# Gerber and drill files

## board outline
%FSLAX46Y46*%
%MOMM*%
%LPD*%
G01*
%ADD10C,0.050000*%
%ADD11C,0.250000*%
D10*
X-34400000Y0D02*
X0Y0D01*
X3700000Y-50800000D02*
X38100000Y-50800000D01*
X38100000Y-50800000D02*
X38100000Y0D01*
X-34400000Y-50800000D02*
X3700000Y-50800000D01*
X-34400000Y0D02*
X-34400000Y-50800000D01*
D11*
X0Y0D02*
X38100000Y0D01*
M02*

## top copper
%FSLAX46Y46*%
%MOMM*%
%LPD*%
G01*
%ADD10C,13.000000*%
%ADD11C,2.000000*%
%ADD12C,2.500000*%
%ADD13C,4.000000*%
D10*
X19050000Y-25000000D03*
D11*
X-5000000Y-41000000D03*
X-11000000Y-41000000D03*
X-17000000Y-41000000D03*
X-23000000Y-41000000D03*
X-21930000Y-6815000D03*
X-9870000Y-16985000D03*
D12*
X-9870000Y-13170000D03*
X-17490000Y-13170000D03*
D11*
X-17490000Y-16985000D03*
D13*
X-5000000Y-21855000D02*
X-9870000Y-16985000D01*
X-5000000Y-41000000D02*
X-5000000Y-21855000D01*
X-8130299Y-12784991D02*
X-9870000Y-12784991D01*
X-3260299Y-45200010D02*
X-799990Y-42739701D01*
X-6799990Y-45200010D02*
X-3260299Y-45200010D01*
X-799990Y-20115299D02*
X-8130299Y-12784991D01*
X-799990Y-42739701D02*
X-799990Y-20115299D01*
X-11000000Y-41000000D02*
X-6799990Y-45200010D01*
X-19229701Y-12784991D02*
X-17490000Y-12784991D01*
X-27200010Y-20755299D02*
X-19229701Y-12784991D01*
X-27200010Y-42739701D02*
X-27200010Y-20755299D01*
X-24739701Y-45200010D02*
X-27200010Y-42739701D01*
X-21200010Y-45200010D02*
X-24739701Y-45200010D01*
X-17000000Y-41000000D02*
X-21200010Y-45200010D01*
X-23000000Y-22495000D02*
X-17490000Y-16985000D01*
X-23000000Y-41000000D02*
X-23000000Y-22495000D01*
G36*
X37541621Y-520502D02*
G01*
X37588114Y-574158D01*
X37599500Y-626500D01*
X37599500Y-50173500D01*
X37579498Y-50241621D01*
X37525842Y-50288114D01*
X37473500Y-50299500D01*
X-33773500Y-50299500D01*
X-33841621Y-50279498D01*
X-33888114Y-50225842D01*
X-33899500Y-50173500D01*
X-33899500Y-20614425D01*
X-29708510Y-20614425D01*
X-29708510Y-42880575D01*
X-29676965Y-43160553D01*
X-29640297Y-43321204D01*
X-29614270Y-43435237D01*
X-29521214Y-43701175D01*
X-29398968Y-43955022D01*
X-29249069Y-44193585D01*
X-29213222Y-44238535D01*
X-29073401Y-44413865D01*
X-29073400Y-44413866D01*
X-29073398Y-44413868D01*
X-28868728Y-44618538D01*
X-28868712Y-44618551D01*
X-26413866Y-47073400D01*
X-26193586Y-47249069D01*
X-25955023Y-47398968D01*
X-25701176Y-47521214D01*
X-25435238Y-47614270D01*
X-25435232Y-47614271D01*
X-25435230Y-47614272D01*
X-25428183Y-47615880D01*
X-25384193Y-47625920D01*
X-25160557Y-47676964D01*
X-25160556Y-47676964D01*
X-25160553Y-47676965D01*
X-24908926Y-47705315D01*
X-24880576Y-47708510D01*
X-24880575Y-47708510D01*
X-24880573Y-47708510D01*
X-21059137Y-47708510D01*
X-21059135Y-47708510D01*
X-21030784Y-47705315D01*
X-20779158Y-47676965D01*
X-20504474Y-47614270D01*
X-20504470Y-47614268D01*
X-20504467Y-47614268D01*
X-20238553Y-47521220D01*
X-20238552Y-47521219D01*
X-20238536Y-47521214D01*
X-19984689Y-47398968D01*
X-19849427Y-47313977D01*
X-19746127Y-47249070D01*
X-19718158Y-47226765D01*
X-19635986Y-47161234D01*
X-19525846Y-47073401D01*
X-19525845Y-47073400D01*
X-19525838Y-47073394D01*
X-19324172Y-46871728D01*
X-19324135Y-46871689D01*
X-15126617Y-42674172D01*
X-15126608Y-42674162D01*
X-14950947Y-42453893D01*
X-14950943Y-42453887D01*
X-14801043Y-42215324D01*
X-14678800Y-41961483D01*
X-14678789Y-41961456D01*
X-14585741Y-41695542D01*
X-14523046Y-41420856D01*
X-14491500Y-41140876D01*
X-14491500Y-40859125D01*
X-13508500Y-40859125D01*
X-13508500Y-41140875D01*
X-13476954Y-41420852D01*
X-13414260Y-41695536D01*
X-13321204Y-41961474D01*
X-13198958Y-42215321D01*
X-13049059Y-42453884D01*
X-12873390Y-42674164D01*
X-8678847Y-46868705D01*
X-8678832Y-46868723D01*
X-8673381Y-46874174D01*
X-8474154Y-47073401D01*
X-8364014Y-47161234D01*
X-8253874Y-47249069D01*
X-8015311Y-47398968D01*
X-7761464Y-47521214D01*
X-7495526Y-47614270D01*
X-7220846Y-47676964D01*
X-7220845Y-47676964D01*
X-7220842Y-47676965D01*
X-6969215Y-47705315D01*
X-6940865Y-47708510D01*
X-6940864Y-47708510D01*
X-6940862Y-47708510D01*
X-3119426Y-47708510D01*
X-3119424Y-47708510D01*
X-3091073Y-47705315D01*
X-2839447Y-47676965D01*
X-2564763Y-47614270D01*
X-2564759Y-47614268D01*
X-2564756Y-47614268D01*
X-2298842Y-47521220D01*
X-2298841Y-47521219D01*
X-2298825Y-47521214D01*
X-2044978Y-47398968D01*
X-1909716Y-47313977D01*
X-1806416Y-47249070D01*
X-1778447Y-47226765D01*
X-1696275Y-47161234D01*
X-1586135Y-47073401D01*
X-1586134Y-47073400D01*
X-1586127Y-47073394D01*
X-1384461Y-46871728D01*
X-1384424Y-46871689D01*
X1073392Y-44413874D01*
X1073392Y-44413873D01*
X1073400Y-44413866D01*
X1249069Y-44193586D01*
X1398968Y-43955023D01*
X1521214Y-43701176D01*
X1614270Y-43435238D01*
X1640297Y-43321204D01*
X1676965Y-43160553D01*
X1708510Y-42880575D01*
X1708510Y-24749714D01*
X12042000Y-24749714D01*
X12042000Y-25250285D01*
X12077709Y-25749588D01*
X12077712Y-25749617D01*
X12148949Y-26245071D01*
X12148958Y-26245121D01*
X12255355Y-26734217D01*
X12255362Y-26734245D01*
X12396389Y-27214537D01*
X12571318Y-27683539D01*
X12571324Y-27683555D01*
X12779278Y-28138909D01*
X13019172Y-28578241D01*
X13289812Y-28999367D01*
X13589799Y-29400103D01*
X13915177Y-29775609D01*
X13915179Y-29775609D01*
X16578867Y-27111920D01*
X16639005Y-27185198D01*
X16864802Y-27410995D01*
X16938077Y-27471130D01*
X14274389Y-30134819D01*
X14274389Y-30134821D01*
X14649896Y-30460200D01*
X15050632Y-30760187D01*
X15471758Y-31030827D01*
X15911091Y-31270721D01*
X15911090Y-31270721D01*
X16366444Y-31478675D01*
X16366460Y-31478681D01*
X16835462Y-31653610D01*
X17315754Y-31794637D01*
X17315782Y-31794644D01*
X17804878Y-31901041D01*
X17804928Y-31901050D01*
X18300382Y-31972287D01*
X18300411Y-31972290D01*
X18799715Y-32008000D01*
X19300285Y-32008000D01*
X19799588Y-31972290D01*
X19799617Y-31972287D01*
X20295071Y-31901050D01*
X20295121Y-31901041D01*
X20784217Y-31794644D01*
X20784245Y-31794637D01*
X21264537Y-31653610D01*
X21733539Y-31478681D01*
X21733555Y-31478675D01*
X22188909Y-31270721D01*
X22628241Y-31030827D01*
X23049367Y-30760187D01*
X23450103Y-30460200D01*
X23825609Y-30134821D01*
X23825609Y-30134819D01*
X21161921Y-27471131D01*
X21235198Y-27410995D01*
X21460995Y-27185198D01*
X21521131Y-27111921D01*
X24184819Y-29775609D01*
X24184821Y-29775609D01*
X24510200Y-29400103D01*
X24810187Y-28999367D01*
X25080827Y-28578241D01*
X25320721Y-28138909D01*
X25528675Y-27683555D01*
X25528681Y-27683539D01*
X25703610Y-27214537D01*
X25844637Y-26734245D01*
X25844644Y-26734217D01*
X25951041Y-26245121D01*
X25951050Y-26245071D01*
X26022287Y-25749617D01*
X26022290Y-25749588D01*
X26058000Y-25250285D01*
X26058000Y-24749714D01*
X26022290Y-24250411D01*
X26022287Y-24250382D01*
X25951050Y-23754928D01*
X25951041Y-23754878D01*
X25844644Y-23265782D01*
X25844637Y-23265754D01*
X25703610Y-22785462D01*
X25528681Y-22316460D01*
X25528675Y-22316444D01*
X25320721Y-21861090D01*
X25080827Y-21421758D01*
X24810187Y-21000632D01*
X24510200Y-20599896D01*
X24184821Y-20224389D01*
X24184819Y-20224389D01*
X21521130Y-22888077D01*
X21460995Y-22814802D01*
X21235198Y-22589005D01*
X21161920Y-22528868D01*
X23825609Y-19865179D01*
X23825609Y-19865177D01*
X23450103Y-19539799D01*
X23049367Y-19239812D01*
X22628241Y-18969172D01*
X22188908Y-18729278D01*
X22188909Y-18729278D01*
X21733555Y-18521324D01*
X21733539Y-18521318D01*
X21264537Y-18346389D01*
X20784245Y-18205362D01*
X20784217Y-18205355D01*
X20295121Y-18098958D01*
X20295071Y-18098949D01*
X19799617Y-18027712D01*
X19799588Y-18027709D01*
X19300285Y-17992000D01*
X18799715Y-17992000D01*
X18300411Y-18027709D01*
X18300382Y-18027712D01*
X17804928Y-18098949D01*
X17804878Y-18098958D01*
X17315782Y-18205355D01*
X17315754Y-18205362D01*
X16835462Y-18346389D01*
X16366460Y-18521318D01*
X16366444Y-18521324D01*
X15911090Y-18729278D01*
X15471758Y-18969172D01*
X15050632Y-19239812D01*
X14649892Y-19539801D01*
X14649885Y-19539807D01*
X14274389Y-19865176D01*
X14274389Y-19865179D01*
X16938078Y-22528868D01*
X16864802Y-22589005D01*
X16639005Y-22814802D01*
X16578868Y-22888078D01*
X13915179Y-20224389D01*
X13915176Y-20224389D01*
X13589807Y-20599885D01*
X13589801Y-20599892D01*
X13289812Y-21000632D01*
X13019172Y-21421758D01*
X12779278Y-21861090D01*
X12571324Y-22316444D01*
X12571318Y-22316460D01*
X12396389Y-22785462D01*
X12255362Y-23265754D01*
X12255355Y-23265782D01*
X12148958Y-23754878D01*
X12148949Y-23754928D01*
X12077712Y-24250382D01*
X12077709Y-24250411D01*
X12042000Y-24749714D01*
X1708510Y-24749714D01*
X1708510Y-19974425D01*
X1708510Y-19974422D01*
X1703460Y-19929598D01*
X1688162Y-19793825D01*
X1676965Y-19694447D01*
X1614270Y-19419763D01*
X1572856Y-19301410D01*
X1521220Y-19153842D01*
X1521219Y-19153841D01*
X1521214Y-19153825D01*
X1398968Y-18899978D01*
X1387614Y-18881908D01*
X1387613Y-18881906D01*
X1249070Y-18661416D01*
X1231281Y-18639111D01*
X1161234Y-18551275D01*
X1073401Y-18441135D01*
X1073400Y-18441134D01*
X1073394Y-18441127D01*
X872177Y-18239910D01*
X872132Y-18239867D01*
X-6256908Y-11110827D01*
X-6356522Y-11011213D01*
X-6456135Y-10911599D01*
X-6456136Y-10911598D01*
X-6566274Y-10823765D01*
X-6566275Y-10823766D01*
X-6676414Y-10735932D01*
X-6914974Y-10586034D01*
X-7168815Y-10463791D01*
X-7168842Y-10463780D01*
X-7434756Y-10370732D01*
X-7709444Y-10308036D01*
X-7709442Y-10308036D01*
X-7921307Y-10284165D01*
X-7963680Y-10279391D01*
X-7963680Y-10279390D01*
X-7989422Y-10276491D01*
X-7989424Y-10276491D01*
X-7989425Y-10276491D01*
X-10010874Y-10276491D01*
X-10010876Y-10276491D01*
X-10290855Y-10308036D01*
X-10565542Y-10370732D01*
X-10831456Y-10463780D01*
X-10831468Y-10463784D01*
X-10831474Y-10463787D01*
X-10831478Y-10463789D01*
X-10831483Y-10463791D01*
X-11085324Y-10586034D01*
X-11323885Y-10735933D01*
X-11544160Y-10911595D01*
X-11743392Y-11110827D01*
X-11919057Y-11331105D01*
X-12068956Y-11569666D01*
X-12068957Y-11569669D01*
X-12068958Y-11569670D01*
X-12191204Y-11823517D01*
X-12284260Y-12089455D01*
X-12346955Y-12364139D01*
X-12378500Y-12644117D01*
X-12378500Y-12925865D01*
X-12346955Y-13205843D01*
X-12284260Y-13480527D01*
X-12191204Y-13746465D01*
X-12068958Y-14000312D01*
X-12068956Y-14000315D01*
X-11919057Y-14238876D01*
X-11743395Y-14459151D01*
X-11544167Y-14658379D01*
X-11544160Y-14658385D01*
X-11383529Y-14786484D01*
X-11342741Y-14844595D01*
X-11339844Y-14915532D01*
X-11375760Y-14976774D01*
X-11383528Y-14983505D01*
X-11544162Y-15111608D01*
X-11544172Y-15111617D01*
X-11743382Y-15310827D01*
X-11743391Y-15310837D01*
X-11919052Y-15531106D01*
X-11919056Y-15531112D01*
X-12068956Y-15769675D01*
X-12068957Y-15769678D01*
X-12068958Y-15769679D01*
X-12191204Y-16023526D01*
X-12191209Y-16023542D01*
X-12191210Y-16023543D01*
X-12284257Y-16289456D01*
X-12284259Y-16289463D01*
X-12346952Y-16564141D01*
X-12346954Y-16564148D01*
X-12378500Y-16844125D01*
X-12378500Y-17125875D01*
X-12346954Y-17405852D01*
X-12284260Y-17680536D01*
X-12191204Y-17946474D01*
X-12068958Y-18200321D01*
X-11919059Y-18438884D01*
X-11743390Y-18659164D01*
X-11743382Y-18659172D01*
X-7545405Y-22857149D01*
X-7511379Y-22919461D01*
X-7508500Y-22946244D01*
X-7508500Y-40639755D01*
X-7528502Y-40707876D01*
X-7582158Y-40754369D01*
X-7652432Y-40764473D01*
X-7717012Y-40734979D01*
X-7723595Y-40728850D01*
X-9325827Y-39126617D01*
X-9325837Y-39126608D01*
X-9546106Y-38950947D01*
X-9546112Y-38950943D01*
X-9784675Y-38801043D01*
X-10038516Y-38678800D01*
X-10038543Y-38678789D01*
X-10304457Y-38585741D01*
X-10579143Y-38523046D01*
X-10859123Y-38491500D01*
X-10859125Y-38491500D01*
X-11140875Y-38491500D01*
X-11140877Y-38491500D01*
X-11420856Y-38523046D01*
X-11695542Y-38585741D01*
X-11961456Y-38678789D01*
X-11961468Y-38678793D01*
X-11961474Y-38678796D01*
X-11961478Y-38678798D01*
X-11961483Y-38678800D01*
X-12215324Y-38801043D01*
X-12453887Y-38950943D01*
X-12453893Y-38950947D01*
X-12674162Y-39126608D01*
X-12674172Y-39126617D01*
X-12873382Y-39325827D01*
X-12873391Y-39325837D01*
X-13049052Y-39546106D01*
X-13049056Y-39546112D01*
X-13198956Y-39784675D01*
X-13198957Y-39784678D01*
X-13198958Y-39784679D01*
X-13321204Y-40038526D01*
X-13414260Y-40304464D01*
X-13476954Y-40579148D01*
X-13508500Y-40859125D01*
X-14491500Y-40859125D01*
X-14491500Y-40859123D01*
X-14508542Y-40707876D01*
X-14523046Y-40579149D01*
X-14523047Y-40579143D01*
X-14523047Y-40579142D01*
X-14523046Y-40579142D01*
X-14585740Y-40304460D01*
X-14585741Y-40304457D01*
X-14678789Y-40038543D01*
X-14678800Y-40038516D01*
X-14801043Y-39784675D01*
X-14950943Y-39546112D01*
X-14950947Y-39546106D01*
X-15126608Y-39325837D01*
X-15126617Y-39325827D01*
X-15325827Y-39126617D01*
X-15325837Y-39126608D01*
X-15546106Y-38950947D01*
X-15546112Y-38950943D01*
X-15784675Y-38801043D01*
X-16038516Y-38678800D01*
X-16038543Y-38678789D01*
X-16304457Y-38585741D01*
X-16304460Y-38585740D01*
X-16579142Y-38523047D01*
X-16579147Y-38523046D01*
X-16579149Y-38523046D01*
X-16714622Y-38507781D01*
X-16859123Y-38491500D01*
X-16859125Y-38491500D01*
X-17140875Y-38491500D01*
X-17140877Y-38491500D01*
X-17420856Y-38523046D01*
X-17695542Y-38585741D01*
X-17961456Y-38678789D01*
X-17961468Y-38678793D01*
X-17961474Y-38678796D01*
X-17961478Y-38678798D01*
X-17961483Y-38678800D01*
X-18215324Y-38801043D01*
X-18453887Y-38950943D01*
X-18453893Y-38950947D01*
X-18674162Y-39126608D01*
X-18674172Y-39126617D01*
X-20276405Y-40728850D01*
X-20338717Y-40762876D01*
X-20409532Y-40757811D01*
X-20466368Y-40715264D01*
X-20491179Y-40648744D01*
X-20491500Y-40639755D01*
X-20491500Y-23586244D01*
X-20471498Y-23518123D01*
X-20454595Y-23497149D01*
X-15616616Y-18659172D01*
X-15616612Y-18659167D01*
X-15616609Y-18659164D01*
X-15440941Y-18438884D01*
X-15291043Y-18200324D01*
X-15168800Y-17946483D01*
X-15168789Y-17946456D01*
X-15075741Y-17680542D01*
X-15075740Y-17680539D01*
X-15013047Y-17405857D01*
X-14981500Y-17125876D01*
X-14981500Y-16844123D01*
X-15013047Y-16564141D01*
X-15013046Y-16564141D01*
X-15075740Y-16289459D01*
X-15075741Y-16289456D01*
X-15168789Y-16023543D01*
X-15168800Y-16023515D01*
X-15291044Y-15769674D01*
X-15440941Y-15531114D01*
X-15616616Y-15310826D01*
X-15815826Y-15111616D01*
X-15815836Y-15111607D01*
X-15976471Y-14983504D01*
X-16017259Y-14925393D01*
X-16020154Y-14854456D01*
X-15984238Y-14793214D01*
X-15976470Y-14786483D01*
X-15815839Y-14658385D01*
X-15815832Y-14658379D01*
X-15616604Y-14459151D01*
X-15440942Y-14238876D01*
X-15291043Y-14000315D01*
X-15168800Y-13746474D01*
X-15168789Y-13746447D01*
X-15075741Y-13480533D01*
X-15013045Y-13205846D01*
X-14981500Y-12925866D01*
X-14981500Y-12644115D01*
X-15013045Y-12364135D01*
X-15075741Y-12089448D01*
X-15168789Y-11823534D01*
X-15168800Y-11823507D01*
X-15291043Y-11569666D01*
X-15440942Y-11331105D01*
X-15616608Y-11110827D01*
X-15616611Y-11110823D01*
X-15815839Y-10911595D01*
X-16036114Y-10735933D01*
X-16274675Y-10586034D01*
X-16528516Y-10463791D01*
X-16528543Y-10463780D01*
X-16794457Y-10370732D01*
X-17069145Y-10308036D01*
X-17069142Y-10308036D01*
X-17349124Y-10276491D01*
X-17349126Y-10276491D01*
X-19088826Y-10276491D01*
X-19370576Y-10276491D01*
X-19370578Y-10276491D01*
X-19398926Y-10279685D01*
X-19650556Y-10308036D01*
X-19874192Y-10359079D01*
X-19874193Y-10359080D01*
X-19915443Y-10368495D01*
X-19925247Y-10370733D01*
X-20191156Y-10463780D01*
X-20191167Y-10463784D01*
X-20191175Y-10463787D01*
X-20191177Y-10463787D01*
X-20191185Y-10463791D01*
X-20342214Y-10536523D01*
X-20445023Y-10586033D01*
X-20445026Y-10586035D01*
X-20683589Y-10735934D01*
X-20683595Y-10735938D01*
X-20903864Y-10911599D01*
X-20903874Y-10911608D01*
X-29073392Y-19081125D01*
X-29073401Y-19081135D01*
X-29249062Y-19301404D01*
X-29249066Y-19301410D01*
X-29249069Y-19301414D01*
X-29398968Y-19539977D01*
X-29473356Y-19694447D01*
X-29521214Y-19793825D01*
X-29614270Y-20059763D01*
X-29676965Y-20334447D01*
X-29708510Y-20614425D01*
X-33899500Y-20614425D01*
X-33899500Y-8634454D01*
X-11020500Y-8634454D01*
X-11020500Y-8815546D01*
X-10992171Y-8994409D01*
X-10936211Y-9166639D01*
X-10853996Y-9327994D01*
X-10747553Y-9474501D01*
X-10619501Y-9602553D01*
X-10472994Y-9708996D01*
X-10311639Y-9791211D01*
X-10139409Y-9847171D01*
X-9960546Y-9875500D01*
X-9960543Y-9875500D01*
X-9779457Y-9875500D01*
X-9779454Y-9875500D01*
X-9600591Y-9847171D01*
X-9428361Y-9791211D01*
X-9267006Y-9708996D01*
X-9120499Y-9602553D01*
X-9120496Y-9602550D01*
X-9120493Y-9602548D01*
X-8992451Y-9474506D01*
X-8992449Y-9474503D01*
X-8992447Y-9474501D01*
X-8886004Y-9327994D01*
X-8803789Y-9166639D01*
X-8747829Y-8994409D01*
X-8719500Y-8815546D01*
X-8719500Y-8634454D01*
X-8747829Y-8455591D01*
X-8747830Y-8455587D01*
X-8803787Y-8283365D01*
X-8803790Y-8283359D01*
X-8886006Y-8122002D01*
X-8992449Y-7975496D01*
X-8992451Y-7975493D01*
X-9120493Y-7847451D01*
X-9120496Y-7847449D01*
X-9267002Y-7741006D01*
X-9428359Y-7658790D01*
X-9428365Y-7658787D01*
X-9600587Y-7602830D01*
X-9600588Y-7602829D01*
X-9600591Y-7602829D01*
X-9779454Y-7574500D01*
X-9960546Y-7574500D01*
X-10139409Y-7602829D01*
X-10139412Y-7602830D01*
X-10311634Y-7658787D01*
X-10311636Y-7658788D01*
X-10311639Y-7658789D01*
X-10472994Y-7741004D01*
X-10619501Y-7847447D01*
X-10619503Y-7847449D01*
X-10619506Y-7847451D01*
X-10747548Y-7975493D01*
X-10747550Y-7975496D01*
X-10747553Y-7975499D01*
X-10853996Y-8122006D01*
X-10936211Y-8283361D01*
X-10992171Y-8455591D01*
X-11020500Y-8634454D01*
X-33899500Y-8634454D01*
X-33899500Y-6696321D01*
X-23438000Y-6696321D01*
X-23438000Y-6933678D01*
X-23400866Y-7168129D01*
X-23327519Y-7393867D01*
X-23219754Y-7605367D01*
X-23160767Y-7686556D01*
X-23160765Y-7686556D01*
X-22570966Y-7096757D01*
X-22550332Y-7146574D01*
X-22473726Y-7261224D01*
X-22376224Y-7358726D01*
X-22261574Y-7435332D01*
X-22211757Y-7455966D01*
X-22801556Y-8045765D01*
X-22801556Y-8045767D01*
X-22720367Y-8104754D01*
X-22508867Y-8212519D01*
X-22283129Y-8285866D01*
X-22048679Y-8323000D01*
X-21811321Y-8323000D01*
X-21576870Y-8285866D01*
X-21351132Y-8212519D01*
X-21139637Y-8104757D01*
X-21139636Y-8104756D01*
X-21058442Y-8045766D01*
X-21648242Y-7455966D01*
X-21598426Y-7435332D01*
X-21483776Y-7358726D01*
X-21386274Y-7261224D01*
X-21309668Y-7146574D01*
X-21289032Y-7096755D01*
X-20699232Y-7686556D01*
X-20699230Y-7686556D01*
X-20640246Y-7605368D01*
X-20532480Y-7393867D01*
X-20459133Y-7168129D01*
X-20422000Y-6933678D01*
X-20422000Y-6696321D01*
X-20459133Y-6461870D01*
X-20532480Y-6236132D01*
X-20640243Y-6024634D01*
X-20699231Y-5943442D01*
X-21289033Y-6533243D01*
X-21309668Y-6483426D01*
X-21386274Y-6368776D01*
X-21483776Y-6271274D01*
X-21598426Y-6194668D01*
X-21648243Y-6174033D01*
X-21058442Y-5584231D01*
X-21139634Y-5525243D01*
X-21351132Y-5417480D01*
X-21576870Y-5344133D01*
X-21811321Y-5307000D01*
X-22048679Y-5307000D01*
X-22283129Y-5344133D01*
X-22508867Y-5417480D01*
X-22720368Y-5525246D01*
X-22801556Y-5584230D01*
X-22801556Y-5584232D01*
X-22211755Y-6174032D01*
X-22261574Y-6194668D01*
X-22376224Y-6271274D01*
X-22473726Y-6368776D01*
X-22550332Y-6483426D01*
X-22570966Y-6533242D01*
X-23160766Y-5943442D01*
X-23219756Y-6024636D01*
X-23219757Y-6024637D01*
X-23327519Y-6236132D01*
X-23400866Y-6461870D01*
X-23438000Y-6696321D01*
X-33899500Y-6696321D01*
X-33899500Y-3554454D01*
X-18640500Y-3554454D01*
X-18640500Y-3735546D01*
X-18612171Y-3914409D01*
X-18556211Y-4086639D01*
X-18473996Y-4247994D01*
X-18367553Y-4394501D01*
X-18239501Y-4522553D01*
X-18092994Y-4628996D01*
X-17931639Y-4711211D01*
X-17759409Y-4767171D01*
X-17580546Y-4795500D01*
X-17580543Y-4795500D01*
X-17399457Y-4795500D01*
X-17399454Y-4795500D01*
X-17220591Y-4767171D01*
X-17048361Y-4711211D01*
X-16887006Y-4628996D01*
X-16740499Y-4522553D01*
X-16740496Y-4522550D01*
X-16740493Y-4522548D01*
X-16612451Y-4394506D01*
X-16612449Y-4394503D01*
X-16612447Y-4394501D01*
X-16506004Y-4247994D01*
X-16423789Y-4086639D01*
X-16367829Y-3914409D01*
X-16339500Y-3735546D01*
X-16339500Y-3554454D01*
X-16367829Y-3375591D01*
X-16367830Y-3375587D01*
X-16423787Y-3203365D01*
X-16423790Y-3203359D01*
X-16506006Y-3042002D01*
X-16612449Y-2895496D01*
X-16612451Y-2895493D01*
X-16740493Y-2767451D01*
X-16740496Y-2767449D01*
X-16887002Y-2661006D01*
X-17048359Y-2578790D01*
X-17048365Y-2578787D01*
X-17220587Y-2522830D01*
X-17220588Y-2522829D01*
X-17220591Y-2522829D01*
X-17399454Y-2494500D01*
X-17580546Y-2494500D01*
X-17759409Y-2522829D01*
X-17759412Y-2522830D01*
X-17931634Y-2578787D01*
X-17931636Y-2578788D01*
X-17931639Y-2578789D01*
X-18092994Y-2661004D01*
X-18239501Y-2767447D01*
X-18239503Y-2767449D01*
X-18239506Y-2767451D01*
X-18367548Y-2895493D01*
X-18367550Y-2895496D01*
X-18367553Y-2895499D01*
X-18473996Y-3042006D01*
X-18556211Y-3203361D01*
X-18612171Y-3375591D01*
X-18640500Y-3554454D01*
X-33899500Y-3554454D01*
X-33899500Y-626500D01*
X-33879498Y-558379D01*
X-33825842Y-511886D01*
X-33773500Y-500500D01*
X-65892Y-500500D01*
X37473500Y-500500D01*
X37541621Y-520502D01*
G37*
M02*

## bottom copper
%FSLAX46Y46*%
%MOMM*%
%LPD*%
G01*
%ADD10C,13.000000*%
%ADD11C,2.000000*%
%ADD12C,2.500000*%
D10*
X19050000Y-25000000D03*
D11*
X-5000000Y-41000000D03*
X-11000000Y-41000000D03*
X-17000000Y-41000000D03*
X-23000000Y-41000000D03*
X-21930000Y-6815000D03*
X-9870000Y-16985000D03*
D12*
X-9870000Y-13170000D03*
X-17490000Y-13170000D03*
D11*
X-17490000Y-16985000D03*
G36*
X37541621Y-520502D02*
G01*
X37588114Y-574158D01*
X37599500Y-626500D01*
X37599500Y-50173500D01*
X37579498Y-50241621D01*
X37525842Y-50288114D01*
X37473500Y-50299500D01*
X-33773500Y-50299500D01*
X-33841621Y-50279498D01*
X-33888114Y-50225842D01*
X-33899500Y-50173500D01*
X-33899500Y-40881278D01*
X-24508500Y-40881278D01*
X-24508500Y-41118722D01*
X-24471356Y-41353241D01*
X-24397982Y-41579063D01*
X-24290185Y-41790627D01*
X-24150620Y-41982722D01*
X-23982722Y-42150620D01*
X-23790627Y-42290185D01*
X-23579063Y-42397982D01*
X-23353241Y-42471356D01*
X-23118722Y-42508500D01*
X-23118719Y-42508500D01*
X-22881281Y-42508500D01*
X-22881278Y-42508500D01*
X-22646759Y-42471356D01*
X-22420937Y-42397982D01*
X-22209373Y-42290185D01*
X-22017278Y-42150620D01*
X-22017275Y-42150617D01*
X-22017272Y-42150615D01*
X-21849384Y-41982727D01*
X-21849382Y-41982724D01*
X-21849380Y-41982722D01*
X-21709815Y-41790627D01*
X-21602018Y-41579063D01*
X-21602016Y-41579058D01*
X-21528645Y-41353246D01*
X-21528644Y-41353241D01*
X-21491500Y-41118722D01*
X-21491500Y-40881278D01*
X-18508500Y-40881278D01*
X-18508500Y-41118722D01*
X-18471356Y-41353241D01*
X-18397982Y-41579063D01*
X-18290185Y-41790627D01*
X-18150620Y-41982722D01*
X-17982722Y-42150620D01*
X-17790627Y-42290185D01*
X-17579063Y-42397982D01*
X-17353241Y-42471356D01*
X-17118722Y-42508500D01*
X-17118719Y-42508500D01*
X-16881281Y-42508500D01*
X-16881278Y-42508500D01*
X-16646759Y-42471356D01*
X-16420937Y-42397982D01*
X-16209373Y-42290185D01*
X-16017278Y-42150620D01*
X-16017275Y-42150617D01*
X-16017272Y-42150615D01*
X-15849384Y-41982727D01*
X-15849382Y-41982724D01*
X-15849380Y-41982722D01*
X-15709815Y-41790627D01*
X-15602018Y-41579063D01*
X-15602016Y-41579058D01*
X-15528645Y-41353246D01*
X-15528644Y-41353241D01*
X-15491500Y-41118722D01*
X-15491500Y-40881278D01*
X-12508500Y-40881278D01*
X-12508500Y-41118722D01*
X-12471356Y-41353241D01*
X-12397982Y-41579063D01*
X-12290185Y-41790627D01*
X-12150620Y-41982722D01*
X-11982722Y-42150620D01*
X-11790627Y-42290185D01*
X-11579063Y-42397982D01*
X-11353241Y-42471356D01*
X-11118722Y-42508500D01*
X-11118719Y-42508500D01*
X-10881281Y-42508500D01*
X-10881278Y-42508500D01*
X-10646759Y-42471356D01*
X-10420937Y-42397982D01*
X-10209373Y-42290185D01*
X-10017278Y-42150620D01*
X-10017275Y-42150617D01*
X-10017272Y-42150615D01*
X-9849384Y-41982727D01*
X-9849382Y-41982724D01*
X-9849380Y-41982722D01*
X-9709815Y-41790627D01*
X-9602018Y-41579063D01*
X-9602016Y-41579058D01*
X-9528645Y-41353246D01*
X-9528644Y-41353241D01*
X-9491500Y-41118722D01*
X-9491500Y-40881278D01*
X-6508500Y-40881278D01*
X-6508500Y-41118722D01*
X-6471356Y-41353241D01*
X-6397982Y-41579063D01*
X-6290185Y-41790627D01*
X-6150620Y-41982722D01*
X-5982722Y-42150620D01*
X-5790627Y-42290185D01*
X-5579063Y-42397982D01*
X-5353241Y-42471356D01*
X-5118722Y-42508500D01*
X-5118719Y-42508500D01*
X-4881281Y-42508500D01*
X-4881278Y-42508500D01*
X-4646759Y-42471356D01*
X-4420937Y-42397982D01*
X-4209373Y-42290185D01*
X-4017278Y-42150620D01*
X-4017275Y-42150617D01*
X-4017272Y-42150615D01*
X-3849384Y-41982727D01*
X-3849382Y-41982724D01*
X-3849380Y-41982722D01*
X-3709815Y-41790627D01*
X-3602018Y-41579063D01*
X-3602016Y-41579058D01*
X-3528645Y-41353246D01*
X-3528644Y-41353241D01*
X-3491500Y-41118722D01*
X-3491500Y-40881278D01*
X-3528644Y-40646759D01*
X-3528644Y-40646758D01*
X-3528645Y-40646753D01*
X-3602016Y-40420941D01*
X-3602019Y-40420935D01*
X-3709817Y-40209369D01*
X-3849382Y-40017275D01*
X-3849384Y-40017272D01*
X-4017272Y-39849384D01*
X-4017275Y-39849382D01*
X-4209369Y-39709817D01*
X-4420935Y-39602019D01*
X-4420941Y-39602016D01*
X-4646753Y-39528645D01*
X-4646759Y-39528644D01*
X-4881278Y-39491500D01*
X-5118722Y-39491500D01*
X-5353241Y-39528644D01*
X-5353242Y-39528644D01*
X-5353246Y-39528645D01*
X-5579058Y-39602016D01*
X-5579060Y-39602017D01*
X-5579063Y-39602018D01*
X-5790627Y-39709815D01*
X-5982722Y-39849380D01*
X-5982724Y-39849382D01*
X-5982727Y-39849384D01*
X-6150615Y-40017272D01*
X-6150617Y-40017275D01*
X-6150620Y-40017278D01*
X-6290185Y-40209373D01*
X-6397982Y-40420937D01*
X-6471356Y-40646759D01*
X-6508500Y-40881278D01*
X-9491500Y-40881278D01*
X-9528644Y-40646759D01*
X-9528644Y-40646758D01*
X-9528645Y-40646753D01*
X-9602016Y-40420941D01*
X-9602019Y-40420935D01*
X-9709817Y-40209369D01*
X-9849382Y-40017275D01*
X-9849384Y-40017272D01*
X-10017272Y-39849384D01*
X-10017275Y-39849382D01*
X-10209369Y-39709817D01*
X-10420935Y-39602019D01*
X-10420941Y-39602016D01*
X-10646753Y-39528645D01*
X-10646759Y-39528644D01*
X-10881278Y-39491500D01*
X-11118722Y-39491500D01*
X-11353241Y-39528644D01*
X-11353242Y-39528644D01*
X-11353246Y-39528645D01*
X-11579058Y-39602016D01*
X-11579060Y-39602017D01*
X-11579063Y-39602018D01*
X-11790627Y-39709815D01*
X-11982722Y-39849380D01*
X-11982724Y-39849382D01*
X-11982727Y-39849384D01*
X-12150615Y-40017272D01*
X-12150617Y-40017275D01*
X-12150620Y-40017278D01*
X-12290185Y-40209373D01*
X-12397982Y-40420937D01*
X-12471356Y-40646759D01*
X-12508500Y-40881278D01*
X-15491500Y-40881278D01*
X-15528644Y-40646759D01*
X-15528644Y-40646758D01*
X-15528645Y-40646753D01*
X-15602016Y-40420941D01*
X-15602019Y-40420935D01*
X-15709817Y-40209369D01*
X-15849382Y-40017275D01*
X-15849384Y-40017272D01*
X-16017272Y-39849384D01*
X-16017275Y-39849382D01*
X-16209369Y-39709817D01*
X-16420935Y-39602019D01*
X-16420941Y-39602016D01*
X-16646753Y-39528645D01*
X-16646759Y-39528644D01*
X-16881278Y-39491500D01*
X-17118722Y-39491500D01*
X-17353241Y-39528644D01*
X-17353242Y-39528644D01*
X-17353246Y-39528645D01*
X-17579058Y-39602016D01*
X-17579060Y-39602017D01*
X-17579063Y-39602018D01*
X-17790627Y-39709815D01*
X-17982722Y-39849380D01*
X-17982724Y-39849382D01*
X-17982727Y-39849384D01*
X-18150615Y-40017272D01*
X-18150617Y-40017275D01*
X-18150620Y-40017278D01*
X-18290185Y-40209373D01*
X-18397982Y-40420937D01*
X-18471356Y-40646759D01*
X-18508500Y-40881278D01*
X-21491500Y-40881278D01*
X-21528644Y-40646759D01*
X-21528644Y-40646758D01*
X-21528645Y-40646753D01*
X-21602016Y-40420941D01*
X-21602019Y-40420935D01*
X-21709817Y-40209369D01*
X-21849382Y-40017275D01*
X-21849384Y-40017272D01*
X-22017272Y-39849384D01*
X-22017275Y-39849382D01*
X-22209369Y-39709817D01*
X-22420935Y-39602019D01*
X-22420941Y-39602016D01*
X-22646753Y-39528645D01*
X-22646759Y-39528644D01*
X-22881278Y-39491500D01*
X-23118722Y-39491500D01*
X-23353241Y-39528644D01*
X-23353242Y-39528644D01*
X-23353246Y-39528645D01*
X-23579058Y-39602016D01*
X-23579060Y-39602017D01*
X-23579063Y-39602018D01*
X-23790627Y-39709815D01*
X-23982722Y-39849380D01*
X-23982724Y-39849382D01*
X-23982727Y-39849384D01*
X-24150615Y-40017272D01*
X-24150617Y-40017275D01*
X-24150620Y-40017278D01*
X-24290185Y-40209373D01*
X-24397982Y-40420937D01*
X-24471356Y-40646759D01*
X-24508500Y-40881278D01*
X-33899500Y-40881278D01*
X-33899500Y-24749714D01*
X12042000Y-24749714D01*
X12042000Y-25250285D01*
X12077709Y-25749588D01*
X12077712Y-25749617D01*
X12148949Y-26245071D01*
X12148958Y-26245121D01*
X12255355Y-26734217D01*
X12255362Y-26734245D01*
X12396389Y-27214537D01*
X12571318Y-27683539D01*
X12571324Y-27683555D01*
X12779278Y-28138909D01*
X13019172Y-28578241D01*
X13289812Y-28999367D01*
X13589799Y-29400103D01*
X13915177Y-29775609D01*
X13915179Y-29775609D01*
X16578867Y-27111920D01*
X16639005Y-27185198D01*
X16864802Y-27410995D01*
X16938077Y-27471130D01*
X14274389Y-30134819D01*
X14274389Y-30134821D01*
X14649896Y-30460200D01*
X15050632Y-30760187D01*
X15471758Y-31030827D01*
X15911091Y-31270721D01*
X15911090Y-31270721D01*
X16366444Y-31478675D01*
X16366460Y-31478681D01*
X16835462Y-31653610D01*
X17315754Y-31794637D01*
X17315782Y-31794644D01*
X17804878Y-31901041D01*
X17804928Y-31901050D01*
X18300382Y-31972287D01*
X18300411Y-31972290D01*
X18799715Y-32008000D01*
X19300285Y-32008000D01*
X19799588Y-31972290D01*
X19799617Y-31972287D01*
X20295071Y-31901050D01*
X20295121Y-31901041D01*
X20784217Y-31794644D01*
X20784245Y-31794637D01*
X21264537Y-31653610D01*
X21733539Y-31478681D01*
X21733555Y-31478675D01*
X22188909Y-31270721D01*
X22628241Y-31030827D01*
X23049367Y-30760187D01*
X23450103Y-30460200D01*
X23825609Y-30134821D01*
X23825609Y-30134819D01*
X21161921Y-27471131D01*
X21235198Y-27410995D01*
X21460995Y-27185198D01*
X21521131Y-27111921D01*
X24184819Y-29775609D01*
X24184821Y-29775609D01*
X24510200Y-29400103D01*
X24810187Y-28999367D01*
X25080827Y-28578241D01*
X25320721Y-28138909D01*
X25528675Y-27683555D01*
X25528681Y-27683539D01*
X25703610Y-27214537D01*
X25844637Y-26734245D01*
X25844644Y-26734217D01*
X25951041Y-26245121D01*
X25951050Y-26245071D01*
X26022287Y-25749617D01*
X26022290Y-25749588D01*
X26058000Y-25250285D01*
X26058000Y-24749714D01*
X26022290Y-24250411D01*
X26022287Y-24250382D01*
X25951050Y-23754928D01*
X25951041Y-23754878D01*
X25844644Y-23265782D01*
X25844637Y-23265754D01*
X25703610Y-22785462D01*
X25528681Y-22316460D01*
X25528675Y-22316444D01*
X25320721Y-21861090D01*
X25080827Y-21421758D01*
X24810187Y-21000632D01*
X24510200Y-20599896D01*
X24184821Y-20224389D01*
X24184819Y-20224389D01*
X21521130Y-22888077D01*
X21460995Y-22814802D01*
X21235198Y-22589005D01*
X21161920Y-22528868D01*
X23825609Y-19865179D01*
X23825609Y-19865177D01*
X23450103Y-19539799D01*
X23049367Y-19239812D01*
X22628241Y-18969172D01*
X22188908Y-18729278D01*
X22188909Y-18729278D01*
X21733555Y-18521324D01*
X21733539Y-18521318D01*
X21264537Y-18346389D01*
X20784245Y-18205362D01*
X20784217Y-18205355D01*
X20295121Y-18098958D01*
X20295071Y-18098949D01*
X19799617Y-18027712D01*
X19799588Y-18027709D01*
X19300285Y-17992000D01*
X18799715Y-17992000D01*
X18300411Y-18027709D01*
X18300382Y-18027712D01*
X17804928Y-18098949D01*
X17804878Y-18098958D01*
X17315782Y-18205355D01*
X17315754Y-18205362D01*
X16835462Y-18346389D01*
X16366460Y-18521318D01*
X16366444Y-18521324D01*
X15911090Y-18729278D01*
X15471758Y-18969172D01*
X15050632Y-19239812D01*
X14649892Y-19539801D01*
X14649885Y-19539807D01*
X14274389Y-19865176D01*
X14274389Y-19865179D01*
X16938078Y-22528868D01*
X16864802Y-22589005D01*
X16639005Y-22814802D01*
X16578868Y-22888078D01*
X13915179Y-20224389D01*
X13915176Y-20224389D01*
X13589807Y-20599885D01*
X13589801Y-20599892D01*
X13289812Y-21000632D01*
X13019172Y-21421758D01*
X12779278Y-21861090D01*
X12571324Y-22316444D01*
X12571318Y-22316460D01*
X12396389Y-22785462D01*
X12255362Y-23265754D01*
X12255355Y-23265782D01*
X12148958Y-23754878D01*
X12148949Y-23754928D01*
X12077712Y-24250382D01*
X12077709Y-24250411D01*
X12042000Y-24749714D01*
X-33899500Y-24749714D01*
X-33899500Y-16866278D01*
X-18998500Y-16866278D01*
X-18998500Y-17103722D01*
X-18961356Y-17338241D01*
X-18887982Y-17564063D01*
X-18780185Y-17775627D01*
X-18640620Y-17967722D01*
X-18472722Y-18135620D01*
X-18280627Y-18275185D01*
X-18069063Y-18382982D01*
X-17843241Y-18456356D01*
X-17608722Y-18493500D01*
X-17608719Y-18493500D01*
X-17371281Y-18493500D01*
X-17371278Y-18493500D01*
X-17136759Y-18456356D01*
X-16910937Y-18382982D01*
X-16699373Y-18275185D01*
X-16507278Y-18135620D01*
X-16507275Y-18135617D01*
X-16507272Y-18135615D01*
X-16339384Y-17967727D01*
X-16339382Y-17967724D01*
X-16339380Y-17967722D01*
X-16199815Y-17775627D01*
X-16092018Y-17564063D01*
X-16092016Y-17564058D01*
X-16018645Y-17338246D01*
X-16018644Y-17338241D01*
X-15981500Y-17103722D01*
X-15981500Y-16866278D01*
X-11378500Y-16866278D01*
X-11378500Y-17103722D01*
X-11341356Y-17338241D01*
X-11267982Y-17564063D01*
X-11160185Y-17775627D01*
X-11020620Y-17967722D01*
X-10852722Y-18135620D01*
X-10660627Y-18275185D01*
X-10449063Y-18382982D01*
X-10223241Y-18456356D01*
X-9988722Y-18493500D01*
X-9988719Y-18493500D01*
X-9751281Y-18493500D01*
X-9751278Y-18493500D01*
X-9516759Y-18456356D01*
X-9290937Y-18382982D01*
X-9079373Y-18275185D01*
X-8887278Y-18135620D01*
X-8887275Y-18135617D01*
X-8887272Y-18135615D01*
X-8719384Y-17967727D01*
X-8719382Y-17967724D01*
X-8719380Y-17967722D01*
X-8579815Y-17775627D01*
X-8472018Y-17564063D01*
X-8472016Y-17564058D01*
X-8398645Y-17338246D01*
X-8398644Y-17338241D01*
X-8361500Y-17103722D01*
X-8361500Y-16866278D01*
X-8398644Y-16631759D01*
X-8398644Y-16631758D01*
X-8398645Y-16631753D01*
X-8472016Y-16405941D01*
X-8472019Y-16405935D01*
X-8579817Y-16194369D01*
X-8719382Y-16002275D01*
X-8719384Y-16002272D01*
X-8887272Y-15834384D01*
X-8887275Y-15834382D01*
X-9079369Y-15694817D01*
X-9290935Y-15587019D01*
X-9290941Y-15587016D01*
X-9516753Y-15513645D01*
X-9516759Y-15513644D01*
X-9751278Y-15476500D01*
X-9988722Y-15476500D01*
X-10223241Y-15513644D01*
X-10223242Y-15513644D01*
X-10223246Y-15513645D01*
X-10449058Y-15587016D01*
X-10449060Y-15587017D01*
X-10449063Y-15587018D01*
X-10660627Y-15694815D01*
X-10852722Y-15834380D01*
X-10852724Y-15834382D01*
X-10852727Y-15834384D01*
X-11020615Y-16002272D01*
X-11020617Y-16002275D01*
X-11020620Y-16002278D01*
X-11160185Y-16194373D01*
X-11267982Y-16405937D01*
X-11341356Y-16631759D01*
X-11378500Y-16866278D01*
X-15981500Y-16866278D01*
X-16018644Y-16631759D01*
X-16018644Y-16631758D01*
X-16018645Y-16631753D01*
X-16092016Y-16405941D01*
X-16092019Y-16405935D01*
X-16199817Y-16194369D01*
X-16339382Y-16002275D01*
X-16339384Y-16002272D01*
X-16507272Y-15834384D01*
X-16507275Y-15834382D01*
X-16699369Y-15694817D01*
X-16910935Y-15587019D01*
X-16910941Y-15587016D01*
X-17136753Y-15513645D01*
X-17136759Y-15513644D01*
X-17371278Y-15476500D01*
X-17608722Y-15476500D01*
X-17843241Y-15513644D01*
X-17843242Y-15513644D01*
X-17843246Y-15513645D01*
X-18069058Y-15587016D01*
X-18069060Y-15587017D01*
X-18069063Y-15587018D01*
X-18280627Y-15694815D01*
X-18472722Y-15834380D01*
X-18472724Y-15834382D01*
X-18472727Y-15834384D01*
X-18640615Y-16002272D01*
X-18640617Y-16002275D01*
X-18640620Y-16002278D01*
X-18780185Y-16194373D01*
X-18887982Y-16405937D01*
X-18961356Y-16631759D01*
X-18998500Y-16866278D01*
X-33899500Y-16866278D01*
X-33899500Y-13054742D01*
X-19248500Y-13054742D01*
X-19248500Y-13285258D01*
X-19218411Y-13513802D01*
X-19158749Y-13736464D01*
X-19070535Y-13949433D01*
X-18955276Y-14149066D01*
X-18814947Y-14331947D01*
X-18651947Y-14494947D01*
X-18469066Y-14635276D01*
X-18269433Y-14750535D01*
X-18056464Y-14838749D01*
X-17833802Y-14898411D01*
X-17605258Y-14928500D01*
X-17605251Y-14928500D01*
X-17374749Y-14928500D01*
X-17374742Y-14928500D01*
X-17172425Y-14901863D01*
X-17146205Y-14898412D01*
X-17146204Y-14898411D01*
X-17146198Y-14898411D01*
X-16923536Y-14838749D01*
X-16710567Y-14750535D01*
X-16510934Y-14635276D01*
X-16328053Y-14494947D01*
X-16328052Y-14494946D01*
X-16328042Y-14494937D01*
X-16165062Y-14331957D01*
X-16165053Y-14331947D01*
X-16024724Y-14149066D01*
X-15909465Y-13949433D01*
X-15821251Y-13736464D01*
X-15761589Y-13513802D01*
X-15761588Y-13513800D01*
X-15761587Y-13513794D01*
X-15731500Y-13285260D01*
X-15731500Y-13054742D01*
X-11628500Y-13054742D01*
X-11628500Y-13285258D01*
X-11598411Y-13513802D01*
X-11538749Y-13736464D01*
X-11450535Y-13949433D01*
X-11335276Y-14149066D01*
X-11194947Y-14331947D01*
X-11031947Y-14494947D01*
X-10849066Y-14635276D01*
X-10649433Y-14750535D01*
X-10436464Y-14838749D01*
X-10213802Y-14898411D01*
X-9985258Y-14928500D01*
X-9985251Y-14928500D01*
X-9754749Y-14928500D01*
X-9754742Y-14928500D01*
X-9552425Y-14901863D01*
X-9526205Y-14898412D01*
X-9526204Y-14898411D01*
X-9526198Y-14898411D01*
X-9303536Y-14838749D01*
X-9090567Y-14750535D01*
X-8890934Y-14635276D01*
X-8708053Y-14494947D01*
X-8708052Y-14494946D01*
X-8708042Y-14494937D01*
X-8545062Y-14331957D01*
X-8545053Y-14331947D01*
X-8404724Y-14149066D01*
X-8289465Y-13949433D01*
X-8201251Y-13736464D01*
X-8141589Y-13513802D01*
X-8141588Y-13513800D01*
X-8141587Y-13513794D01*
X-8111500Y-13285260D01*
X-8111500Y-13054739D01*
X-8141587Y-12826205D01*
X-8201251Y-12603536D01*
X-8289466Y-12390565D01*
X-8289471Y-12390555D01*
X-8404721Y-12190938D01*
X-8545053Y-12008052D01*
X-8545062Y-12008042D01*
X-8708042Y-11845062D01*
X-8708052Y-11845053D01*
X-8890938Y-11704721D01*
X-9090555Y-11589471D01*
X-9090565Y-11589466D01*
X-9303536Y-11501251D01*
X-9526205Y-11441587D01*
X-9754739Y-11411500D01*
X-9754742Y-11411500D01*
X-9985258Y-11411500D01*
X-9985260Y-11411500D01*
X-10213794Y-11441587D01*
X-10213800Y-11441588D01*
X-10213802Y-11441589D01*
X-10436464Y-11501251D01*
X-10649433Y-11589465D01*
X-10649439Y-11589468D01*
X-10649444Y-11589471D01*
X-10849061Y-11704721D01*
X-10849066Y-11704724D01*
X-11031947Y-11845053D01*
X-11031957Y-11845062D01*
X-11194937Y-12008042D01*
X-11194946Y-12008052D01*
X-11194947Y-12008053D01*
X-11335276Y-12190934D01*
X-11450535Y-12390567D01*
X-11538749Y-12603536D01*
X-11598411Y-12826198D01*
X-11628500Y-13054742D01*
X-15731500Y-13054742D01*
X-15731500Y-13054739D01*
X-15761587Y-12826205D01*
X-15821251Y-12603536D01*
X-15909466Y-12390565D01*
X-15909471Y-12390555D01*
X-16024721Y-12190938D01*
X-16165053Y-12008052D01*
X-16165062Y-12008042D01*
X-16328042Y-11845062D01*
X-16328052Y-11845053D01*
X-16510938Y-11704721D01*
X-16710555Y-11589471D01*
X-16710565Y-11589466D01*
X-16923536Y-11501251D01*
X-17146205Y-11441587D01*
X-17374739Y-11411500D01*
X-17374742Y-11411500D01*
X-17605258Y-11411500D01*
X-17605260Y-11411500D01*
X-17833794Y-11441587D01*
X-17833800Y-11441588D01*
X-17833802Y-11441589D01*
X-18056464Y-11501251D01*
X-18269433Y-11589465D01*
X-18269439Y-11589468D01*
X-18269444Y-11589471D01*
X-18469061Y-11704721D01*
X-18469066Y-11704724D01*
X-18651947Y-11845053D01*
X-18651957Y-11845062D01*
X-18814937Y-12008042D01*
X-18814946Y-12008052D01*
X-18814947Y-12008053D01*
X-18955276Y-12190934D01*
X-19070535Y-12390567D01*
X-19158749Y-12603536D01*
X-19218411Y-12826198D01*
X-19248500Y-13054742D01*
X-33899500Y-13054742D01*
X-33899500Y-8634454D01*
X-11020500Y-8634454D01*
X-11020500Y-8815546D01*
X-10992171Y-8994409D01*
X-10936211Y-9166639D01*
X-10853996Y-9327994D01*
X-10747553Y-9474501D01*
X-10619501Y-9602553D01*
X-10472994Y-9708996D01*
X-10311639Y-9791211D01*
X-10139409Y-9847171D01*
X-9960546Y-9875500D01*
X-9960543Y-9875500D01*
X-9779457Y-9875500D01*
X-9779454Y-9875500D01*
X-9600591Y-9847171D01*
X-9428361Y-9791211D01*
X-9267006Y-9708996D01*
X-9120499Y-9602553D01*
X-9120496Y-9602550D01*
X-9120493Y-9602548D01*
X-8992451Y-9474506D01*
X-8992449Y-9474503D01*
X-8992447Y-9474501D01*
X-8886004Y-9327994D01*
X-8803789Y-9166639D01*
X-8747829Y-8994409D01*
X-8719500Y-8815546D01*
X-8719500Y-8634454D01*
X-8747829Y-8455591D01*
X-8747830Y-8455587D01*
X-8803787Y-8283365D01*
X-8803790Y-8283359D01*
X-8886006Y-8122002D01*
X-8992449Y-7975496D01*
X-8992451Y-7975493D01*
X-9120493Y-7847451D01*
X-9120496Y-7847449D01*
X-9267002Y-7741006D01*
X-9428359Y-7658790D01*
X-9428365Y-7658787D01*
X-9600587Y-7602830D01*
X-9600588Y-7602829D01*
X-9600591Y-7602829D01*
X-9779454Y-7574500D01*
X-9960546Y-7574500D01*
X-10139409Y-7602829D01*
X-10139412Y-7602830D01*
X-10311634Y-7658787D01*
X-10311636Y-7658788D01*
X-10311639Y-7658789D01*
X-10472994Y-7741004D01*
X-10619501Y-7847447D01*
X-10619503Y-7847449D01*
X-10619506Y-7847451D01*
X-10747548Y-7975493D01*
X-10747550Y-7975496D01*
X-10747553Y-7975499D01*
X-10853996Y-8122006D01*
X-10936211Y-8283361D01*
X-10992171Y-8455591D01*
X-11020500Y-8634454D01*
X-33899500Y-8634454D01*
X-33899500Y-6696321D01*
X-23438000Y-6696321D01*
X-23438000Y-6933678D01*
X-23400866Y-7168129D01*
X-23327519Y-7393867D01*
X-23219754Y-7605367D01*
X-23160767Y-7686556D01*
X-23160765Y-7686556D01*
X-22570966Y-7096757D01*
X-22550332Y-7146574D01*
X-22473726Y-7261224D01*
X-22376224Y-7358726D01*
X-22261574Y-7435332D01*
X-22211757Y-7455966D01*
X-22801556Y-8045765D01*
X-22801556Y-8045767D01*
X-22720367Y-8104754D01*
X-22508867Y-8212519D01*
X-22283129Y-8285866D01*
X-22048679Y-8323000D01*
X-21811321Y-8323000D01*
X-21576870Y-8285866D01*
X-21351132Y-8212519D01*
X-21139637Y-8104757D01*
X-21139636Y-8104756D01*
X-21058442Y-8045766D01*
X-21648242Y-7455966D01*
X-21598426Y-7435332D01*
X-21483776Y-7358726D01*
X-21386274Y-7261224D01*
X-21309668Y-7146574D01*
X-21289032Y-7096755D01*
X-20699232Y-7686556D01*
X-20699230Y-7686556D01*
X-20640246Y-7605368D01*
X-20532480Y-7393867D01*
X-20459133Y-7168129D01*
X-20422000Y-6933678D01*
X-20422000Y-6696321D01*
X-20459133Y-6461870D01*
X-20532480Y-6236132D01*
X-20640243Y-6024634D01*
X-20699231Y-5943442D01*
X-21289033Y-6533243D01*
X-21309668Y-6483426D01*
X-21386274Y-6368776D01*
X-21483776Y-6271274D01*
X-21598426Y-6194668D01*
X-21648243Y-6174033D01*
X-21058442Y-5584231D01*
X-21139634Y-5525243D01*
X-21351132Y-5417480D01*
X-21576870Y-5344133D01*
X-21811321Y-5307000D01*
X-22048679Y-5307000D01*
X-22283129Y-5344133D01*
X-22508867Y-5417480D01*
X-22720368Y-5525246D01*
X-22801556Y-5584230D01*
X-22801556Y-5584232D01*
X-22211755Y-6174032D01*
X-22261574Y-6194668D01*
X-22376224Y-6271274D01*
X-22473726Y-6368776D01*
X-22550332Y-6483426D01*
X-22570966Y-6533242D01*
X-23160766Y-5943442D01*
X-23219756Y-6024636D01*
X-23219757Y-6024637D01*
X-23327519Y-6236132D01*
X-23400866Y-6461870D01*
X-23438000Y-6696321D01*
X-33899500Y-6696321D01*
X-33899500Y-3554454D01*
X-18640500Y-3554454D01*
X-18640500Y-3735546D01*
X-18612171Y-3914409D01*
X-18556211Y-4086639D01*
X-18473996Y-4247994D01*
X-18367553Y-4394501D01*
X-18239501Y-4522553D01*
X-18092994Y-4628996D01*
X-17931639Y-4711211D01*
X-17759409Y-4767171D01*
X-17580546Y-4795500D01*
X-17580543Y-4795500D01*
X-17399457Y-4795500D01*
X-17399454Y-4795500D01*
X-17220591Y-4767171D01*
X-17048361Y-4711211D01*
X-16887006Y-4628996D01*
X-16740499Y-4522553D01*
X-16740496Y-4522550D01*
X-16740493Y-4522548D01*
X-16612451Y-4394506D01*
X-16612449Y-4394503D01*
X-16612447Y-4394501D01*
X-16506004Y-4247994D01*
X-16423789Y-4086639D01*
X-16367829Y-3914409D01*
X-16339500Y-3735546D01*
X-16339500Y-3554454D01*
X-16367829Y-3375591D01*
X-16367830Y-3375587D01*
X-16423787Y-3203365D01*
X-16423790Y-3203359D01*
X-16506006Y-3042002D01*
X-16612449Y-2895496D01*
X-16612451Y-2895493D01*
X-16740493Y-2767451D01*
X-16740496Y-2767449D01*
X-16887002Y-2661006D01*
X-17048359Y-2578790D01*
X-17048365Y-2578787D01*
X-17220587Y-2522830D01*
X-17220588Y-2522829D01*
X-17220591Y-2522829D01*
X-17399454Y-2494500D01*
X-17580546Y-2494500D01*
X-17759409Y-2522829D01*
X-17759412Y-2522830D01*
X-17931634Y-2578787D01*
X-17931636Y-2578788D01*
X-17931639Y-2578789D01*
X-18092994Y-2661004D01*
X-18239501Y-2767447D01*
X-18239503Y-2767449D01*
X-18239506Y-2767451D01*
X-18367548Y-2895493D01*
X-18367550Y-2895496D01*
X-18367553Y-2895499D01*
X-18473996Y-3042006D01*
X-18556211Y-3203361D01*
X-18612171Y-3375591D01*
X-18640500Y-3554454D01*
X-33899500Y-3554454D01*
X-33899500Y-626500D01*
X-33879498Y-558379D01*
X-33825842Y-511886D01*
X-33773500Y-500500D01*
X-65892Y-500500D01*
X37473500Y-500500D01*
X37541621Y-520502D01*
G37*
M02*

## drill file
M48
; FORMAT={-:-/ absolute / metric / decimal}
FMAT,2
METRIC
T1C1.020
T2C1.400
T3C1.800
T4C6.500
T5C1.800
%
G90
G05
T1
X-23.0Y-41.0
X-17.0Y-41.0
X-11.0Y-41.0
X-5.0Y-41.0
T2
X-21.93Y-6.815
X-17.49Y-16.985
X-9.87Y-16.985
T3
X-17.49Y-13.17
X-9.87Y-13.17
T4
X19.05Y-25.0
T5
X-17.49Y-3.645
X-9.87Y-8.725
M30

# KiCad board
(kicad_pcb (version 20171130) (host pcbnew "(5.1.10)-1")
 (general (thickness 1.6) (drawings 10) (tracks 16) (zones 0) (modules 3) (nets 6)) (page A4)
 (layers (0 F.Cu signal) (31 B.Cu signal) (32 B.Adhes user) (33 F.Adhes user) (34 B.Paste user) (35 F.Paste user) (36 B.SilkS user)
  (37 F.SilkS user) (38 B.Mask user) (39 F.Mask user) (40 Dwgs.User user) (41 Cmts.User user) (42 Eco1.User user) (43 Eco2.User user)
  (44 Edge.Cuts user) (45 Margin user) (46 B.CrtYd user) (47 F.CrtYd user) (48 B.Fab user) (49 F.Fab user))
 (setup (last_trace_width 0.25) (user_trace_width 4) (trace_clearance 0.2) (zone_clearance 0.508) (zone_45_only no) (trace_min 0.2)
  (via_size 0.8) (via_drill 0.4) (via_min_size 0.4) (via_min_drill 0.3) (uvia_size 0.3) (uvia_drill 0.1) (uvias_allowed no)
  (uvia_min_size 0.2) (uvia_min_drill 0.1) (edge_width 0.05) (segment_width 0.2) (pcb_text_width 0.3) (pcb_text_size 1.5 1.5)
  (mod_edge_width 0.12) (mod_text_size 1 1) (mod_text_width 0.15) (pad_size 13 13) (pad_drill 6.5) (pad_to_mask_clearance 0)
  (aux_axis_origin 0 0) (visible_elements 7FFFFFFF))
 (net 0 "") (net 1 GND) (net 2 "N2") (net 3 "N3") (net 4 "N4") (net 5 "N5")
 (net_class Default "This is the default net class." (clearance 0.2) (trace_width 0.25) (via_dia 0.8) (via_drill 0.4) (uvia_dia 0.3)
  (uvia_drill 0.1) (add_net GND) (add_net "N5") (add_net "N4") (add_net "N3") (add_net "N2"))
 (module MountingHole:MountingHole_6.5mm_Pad (layer F.Cu) (at 19.05 25)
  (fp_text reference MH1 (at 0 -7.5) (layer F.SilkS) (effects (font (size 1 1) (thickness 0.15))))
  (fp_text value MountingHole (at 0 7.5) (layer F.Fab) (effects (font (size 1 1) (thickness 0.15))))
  (pad 1 thru_hole circle (at 0 0) (size 13 13) (drill 6.5) (layers *.Cu *.Mask) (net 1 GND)))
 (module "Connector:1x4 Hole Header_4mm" (layer F.Cu) (at -23 41)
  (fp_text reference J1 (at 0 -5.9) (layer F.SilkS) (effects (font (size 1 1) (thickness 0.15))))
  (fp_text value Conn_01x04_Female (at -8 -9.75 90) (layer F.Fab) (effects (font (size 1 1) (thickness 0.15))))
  (pad 4 thru_hole circle (at 18 0) (size 2 2) (drill 1.02) (layers *.Cu *.Mask) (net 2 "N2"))
  (pad 3 thru_hole circle (at 12 0) (size 2 2) (drill 1.02) (layers *.Cu *.Mask) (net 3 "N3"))
  (pad 2 thru_hole circle (at 6 0) (size 2 2) (drill 1.02) (layers *.Cu *.Mask) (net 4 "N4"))
  (pad 1 thru_hole circle (at 0 0) (size 2 2) (drill 1.02) (layers *.Cu *.Mask) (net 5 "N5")))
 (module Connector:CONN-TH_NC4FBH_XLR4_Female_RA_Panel (layer F.Cu) (at -15.9 11.9 180)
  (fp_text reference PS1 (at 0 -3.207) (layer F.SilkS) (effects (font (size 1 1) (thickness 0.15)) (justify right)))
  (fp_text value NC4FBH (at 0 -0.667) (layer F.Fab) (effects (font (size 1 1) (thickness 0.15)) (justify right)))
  (pad "" np_thru_hole circle (at -6.03 3.175 180) (size 1.8 1.8) (drill 1.8) (layers *.Cu *.Mask))
  (pad "" np_thru_hole circle (at 1.59 8.255 180) (size 1.8 1.8) (drill 1.8) (layers *.Cu *.Mask))
  (pad 5 thru_hole circle (at 6.03 5.085) (size 2 2) (drill 1.4) (layers *.Cu *.Mask) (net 1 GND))
  (pad 4 thru_hole circle (at -6.03 -5.085) (size 2 2) (drill 1.4) (layers *.Cu *.Mask) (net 2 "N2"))
  (pad 3 thru_hole circle (at -6.03 -1.27) (size 2.5 2.5) (drill 1.8) (layers *.Cu *.Mask) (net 3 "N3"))
  (pad 2 thru_hole circle (at 1.59 -1.27) (size 2.5 2.5) (drill 1.8) (layers *.Cu *.Mask) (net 4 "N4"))
  (pad 1 thru_hole circle (at 1.59 -5.085) (size 2 2) (drill 1.4) (layers *.Cu *.Mask) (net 5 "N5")))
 (gr_line (start -34.4 0) (end 0 0) (layer Edge.Cuts) (width 0.05))
 (gr_line (start 3.7 50.8) (end 38.1 50.8) (layer Edge.Cuts) (width 0.05))
 (gr_line (start 38.1 50.8) (end 38.1 0) (layer Edge.Cuts) (width 0.05))
 (gr_line (start -34.4 50.8) (end 3.7 50.8) (layer Edge.Cuts) (width 0.05))
 (gr_line (start -34.4 0) (end -34.4 50.8) (layer Edge.Cuts) (width 0.05))
 (gr_line (start 0 0) (end 38.1 0) (layer Edge.Cuts) (width 0.25))
 (segment (start -5 21.855) (end -9.87 16.985) (width 4) (layer F.Cu) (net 2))
 (segment (start -5 41) (end -5 21.855) (width 4) (layer F.Cu) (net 2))
 (segment (start -8.130299 12.784991) (end -9.87 12.784991) (width 4) (layer F.Cu) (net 3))
 (segment (start -3.260299 45.20001) (end -0.79999 42.739701) (width 4) (layer F.Cu) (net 3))
 (segment (start -6.79999 45.20001) (end -3.260299 45.20001) (width 4) (layer F.Cu) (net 3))
 (segment (start -0.79999 20.115299) (end -8.130299 12.784991) (width 4) (layer F.Cu) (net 3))
 (segment (start -0.79999 42.739701) (end -0.79999 20.115299) (width 4) (layer F.Cu) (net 3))
 (segment (start -11 41) (end -6.79999 45.20001) (width 4) (layer F.Cu) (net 3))
 (segment (start -19.229701 12.784991) (end -17.49 12.784991) (width 4) (layer F.Cu) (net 4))
 (segment (start -27.20001 20.755299) (end -19.229701 12.784991) (width 4) (layer F.Cu) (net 4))
 (segment (start -27.20001 42.739701) (end -27.20001 20.755299) (width 4) (layer F.Cu) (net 4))
 (segment (start -24.739701 45.20001) (end -27.20001 42.739701) (width 4) (layer F.Cu) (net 4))
 (segment (start -21.20001 45.20001) (end -24.739701 45.20001) (width 4) (layer F.Cu) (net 4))
 (segment (start -17 41) (end -21.20001 45.20001) (width 4) (layer F.Cu) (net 4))
 (segment (start -23 22.495) (end -17.49 16.985) (width 4) (layer F.Cu) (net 5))
 (segment (start -23 41) (end -23 22.495) (width 4) (layer F.Cu) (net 5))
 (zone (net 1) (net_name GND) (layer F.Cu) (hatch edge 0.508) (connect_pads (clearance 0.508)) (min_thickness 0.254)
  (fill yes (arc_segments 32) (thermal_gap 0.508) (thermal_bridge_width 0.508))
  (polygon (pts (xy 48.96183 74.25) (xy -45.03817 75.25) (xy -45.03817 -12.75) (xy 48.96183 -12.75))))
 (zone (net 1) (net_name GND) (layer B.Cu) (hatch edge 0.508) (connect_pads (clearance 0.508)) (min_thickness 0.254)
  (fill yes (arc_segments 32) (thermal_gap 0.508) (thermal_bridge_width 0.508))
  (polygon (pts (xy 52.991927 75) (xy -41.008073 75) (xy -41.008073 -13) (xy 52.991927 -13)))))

